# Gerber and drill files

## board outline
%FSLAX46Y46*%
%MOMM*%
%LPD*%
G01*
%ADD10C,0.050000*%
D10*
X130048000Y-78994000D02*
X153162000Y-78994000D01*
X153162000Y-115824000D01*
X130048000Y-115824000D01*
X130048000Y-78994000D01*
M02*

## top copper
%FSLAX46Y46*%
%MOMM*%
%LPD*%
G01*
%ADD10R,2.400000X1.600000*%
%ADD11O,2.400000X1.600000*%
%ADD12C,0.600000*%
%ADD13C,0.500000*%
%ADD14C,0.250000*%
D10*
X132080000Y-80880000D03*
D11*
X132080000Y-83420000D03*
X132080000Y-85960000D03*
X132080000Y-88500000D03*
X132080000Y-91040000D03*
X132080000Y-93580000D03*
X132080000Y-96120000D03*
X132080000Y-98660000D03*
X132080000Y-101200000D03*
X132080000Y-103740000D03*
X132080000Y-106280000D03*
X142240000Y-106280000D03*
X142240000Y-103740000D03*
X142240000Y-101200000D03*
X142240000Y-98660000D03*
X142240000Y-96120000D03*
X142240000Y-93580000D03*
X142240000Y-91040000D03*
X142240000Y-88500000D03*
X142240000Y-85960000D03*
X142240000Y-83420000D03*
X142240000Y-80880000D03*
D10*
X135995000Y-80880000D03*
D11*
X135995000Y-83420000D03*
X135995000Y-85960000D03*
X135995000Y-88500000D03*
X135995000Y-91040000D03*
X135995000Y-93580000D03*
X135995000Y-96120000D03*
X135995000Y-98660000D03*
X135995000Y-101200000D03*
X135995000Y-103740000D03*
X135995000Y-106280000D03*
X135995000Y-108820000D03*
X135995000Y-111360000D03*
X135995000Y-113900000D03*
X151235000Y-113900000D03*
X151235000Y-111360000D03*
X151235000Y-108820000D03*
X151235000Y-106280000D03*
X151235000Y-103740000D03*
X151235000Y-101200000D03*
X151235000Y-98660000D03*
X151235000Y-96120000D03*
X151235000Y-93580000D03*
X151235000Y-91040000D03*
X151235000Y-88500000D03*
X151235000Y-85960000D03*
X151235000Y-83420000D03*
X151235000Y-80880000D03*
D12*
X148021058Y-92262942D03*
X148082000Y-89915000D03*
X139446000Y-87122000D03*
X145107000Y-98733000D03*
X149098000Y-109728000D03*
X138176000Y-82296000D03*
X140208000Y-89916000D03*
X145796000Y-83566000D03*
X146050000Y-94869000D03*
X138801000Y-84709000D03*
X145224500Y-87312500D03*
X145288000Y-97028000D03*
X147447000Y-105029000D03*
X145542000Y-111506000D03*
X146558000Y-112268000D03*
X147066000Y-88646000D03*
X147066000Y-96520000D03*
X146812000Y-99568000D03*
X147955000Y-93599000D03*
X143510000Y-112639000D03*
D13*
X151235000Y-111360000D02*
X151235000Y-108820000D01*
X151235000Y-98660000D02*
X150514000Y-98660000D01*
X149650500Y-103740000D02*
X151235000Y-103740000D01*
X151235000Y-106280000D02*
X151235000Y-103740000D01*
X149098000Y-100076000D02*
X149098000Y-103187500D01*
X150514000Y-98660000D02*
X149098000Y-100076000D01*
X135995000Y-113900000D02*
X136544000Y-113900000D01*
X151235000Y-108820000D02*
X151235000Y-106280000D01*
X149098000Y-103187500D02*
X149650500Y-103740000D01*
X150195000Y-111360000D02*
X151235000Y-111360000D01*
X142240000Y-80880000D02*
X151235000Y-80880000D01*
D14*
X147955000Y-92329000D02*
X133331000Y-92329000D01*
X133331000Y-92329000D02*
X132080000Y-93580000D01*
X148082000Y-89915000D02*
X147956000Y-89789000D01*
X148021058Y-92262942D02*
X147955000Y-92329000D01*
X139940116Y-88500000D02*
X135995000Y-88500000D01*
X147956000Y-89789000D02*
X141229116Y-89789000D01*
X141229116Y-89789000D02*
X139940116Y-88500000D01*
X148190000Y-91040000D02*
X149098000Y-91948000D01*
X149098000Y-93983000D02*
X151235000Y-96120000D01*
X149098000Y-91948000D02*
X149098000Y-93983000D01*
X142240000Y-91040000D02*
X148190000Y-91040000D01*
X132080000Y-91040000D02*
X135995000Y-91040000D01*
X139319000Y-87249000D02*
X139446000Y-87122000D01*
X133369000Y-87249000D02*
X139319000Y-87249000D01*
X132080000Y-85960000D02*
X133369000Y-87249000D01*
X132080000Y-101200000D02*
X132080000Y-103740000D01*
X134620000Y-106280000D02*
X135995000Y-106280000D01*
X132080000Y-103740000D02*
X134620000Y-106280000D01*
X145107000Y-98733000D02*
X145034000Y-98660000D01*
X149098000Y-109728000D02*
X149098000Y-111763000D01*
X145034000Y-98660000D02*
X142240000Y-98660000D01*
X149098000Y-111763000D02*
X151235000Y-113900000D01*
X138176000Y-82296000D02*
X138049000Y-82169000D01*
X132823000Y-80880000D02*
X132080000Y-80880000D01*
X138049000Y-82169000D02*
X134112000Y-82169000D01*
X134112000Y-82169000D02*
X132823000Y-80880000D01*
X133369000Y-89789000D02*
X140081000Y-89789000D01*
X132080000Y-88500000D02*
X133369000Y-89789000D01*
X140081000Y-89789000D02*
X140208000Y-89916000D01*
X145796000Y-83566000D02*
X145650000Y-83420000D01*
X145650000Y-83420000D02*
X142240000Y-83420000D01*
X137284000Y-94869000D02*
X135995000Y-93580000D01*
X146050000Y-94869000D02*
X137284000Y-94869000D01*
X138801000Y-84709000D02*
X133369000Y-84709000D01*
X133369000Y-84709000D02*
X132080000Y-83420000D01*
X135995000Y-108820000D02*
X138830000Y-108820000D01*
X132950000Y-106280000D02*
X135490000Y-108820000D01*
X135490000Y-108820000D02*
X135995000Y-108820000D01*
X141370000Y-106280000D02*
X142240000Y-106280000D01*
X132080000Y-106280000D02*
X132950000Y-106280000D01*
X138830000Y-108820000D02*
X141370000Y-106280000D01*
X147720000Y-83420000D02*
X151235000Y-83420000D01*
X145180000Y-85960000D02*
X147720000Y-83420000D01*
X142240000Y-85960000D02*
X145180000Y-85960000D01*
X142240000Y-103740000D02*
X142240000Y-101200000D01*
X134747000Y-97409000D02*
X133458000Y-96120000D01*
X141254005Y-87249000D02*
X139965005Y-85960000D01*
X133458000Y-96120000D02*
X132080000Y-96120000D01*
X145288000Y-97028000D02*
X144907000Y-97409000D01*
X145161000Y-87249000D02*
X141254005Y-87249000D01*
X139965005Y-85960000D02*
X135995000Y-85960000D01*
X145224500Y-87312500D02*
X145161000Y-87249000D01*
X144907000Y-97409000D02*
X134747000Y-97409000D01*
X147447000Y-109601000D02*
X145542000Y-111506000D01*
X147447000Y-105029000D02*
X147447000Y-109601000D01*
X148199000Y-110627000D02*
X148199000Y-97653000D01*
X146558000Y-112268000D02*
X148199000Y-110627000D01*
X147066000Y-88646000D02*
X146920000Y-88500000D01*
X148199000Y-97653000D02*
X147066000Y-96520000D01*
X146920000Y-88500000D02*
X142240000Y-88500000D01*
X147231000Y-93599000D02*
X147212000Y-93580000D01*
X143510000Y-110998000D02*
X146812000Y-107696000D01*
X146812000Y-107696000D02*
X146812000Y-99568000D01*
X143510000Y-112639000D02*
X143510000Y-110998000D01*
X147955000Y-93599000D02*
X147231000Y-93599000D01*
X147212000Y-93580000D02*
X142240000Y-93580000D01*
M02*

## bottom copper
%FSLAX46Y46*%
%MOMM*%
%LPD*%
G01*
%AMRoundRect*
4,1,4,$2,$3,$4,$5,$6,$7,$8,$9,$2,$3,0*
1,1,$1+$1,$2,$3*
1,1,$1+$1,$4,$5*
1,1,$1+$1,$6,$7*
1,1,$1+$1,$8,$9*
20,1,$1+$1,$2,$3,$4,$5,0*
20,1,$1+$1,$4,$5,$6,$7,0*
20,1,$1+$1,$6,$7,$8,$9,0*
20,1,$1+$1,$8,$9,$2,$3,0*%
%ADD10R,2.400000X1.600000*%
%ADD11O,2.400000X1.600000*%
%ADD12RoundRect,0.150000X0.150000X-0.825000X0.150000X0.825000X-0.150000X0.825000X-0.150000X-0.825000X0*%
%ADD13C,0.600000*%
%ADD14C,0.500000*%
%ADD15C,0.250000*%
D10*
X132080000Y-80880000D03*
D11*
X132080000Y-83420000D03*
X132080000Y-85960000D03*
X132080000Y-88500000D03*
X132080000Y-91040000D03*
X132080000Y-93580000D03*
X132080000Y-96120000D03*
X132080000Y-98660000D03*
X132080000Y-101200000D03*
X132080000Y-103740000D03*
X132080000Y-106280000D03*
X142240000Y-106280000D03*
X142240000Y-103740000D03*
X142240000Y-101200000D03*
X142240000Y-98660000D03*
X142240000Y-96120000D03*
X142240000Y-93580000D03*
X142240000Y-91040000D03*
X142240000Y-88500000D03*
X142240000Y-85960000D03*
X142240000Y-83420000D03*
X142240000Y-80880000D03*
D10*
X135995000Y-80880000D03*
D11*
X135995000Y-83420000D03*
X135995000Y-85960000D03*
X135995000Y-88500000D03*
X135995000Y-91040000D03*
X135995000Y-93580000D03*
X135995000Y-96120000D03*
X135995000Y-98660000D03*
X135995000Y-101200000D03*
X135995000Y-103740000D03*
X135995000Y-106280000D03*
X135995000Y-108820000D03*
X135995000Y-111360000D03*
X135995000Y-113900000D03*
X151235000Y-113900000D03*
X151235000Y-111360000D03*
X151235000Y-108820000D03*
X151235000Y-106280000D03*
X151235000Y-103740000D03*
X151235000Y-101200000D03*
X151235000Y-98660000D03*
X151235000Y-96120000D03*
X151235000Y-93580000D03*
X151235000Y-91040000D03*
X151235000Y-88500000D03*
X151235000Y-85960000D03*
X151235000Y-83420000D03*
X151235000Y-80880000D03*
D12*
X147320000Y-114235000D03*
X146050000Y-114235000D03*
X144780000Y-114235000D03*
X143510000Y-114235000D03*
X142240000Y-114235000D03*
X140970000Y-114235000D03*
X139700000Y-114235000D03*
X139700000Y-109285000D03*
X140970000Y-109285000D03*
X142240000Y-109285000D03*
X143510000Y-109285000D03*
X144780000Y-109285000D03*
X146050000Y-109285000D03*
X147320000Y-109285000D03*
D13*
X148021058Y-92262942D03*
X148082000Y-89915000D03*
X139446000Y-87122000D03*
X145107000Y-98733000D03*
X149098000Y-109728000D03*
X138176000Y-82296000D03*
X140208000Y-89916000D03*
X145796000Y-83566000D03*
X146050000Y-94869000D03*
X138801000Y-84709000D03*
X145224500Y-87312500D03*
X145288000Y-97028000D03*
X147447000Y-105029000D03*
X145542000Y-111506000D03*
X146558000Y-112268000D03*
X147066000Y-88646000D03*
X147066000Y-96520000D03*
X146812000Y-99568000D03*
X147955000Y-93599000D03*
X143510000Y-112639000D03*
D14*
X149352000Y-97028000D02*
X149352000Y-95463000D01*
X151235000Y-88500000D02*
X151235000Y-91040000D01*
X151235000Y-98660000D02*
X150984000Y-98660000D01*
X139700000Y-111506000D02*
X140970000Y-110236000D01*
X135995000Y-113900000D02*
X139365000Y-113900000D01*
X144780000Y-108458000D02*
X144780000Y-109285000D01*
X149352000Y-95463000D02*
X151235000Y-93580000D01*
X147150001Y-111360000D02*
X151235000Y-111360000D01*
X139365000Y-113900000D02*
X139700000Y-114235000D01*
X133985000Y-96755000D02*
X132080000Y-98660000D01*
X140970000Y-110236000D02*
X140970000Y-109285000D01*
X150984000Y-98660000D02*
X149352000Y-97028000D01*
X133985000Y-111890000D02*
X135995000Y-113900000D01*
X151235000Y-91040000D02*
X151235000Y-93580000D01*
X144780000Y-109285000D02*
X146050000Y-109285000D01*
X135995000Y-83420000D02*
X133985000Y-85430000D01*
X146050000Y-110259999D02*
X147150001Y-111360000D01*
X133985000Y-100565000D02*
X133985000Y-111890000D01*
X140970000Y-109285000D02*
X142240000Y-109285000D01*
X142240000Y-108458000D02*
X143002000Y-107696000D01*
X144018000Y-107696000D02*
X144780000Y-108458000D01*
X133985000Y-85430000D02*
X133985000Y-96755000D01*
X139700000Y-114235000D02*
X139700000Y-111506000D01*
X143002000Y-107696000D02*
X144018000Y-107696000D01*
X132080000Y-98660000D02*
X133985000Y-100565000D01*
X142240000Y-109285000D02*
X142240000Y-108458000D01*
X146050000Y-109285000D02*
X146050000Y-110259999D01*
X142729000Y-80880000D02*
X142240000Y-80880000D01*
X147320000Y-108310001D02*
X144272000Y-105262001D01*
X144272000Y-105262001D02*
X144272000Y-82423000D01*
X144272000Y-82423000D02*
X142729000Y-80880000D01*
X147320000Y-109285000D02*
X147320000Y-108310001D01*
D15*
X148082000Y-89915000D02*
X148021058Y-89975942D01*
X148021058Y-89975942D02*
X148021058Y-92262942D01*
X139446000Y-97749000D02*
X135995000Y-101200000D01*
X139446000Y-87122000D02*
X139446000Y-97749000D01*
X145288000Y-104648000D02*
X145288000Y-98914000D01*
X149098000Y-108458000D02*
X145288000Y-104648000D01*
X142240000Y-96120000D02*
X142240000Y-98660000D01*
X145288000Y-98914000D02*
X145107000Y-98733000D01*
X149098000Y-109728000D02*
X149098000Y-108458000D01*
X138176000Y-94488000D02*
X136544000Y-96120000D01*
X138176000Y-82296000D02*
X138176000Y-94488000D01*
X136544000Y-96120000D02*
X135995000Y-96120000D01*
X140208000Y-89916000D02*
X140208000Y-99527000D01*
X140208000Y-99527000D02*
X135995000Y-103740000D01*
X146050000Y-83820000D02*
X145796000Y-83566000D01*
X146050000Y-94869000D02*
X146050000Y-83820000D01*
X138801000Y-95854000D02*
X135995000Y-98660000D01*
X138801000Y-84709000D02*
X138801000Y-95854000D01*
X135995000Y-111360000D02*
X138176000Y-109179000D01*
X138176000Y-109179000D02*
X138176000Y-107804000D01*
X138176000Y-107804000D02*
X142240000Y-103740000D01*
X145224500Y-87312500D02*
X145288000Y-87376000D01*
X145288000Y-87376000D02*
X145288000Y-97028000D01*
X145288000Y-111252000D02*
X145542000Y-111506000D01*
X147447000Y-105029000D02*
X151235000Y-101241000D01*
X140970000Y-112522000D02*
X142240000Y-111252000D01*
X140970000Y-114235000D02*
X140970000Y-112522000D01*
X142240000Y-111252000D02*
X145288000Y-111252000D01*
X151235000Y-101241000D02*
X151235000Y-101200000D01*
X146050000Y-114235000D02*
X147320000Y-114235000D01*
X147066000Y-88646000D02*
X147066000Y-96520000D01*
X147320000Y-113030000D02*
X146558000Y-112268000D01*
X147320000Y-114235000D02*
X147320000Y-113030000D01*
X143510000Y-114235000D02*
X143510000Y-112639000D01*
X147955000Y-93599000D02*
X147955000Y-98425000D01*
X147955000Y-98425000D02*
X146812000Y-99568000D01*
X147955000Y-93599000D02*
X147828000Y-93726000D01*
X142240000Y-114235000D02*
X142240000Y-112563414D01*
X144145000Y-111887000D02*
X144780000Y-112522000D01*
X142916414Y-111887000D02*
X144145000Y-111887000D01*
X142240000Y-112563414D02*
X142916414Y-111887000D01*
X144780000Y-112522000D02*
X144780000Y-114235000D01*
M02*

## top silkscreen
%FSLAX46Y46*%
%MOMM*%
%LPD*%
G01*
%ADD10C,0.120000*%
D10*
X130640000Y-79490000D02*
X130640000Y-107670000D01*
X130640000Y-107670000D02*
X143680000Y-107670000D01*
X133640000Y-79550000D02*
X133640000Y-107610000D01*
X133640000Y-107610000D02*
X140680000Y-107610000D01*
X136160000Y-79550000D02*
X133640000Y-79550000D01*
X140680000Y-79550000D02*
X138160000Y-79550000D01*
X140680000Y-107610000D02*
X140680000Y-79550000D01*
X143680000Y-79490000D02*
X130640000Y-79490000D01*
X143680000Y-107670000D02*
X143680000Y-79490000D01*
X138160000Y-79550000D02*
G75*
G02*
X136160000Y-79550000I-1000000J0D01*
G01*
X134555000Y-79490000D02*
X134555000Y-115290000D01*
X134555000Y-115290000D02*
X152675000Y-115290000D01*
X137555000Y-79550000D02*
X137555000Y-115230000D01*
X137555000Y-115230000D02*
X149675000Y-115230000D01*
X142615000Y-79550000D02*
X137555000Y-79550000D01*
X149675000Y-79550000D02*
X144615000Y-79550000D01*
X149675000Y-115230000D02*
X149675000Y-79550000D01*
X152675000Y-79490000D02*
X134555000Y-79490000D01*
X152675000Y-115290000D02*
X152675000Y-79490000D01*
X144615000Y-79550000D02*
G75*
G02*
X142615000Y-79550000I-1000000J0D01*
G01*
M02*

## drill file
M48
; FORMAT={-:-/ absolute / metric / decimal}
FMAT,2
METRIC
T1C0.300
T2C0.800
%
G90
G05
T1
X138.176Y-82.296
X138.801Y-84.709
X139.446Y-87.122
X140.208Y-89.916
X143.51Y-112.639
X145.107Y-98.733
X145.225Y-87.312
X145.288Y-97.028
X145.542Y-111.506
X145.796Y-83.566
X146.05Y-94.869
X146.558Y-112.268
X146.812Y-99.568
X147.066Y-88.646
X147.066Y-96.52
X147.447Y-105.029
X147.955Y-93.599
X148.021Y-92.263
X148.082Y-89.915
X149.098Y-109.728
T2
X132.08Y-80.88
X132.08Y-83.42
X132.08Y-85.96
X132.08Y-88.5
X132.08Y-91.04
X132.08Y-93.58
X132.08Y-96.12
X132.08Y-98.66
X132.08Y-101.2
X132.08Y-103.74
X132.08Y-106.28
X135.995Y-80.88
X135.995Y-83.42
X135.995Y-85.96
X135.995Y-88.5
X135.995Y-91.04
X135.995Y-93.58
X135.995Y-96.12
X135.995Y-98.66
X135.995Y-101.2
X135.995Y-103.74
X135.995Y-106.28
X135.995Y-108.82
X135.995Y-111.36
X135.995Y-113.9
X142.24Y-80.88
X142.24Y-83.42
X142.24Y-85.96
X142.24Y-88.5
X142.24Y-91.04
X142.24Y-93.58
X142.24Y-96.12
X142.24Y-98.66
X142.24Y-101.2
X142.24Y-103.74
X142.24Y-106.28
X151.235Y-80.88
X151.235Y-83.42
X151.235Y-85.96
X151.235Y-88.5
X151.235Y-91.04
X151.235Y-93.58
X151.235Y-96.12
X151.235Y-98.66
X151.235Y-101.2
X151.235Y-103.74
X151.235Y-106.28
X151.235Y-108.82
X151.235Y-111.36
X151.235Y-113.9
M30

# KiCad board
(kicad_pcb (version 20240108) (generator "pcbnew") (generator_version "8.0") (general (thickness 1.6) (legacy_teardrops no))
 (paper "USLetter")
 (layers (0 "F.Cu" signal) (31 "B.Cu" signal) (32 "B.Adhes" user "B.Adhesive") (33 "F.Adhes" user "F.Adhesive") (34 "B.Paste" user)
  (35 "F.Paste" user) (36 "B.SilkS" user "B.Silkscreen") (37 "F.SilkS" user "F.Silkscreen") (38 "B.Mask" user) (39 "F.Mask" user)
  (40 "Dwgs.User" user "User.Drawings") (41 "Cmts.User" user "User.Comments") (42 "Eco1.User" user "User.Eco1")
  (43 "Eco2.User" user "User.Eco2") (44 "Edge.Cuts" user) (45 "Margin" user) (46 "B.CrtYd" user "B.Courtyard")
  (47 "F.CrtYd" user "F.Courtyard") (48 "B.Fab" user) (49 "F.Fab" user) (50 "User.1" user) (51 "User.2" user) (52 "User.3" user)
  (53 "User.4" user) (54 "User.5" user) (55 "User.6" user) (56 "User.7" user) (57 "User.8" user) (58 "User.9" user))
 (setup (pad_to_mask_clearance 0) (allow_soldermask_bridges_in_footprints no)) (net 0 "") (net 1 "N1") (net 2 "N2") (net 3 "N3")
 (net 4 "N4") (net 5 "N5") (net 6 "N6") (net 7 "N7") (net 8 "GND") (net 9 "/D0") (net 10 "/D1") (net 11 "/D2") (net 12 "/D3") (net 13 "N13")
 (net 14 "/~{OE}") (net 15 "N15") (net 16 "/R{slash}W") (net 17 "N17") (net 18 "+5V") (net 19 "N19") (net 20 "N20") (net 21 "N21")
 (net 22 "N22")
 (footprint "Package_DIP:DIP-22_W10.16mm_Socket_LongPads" (layer "F.Cu") (at 132.08 80.88)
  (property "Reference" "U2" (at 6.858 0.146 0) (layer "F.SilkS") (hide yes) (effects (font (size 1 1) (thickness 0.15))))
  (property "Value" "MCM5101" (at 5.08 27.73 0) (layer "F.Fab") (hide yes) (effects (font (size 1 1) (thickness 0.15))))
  (fp_line (start -1.44 -1.39) (end -1.44 26.79) (stroke (width 0.12) (type solid)) (layer "F.SilkS"))
  (fp_line (start -1.44 26.79) (end 11.6 26.79) (stroke (width 0.12) (type solid)) (layer "F.SilkS"))
  (fp_line (start 1.56 -1.33) (end 1.56 26.73) (stroke (width 0.12) (type solid)) (layer "F.SilkS"))
  (fp_line (start 1.56 26.73) (end 8.6 26.73) (stroke (width 0.12) (type solid)) (layer "F.SilkS"))
  (fp_line (start 4.08 -1.33) (end 1.56 -1.33) (stroke (width 0.12) (type solid)) (layer "F.SilkS"))
  (fp_line (start 8.6 -1.33) (end 6.08 -1.33) (stroke (width 0.12) (type solid)) (layer "F.SilkS"))
  (fp_line (start 8.6 26.73) (end 8.6 -1.33) (stroke (width 0.12) (type solid)) (layer "F.SilkS"))
  (fp_line (start 11.6 -1.39) (end -1.44 -1.39) (stroke (width 0.12) (type solid)) (layer "F.SilkS"))
  (fp_line (start 11.6 26.79) (end 11.6 -1.39) (stroke (width 0.12) (type solid)) (layer "F.SilkS"))
  (fp_arc (start 6.08 -1.33) (mid 5.08 -0.33) (end 4.08 -1.33) (stroke (width 0.12) (type solid)) (layer "F.SilkS"))
  (pad "1" thru_hole rect (at 0 0) (size 2.4 1.6) (drill 0.8) (layers "*.Cu" "*.Mask") (remove_unused_layers no) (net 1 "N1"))
  (pad "2" thru_hole oval (at 0 2.54) (size 2.4 1.6) (drill 0.8) (layers "*.Cu" "*.Mask") (remove_unused_layers no) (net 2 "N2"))
  (pad "3" thru_hole oval (at 0 5.08) (size 2.4 1.6) (drill 0.8) (layers "*.Cu" "*.Mask") (remove_unused_layers no) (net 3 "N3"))
  (pad "4" thru_hole oval (at 0 7.62) (size 2.4 1.6) (drill 0.8) (layers "*.Cu" "*.Mask") (remove_unused_layers no) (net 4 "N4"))
  (pad "5" thru_hole oval (at 0 10.16) (size 2.4 1.6) (drill 0.8) (layers "*.Cu" "*.Mask") (remove_unused_layers no) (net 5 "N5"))
  (pad "6" thru_hole oval (at 0 12.7) (size 2.4 1.6) (drill 0.8) (layers "*.Cu" "*.Mask") (remove_unused_layers no) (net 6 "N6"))
  (pad "7" thru_hole oval (at 0 15.24) (size 2.4 1.6) (drill 0.8) (layers "*.Cu" "*.Mask") (remove_unused_layers no) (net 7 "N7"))
  (pad "8" thru_hole oval (at 0 17.78) (size 2.4 1.6) (drill 0.8) (layers "*.Cu" "*.Mask") (remove_unused_layers no) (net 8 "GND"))
  (pad "9" thru_hole oval (at 0 20.32) (size 2.4 1.6) (drill 0.8) (layers "*.Cu" "*.Mask") (remove_unused_layers no) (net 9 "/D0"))
  (pad "10" thru_hole oval (at 0 22.86) (size 2.4 1.6) (drill 0.8) (layers "*.Cu" "*.Mask") (remove_unused_layers no) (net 9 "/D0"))
  (pad "11" thru_hole oval (at 0 25.4) (size 2.4 1.6) (drill 0.8) (layers "*.Cu" "*.Mask") (remove_unused_layers no) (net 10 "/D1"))
  (pad "12" thru_hole oval (at 10.16 25.4) (size 2.4 1.6) (drill 0.8) (layers "*.Cu" "*.Mask") (remove_unused_layers no) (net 10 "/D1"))
  (pad "13" thru_hole oval (at 10.16 22.86) (size 2.4 1.6) (drill 0.8) (layers "*.Cu" "*.Mask") (remove_unused_layers no) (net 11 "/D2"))
  (pad "14" thru_hole oval (at 10.16 20.32) (size 2.4 1.6) (drill 0.8) (layers "*.Cu" "*.Mask") (remove_unused_layers no) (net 11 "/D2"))
  (pad "15" thru_hole oval (at 10.16 17.78) (size 2.4 1.6) (drill 0.8) (layers "*.Cu" "*.Mask") (remove_unused_layers no) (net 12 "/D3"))
  (pad "16" thru_hole oval (at 10.16 15.24) (size 2.4 1.6) (drill 0.8) (layers "*.Cu" "*.Mask") (remove_unused_layers no) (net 12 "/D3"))
  (pad "17" thru_hole oval (at 10.16 12.7) (size 2.4 1.6) (drill 0.8) (layers "*.Cu" "*.Mask") (remove_unused_layers no) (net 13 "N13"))
  (pad "18" thru_hole oval (at 10.16 10.16) (size 2.4 1.6) (drill 0.8) (layers "*.Cu" "*.Mask") (remove_unused_layers no) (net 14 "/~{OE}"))
  (pad "19" thru_hole oval (at 10.16 7.62) (size 2.4 1.6) (drill 0.8) (layers "*.Cu" "*.Mask") (remove_unused_layers no) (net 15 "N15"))
  (pad "20" thru_hole oval (at 10.16 5.08) (size 2.4 1.6) (drill 0.8) (layers "*.Cu" "*.Mask") (remove_unused_layers no)
   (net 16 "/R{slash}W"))
  (pad "21" thru_hole oval (at 10.16 2.54) (size 2.4 1.6) (drill 0.8) (layers "*.Cu" "*.Mask") (remove_unused_layers no) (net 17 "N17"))
  (pad "22" thru_hole oval (at 10.16 0) (size 2.4 1.6) (drill 0.8) (layers "*.Cu" "*.Mask") (remove_unused_layers no) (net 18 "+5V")))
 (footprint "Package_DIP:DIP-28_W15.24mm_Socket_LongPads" (layer "F.Cu") (at 135.995 80.88)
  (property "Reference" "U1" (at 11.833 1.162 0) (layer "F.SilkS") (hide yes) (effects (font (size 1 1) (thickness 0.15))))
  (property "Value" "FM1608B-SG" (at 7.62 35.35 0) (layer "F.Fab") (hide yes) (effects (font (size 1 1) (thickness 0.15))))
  (fp_line (start -1.44 -1.39) (end -1.44 34.41) (stroke (width 0.12) (type solid)) (layer "F.SilkS"))
  (fp_line (start -1.44 34.41) (end 16.68 34.41) (stroke (width 0.12) (type solid)) (layer "F.SilkS"))
  (fp_line (start 1.56 -1.33) (end 1.56 34.35) (stroke (width 0.12) (type solid)) (layer "F.SilkS"))
  (fp_line (start 1.56 34.35) (end 13.68 34.35) (stroke (width 0.12) (type solid)) (layer "F.SilkS"))
  (fp_line (start 6.62 -1.33) (end 1.56 -1.33) (stroke (width 0.12) (type solid)) (layer "F.SilkS"))
  (fp_line (start 13.68 -1.33) (end 8.62 -1.33) (stroke (width 0.12) (type solid)) (layer "F.SilkS"))
  (fp_line (start 13.68 34.35) (end 13.68 -1.33) (stroke (width 0.12) (type solid)) (layer "F.SilkS"))
  (fp_line (start 16.68 -1.39) (end -1.44 -1.39) (stroke (width 0.12) (type solid)) (layer "F.SilkS"))
  (fp_line (start 16.68 34.41) (end 16.68 -1.39) (stroke (width 0.12) (type solid)) (layer "F.SilkS"))
  (fp_arc (start 8.62 -1.33) (mid 7.62 -0.33) (end 6.62 -1.33) (stroke (width 0.12) (type solid)) (layer "F.SilkS"))
  (pad "1" thru_hole rect (at 0 0) (size 2.4 1.6) (drill 0.8) (layers "*.Cu" "*.Mask") (remove_unused_layers no))
  (pad "2" thru_hole oval (at 0 2.54) (size 2.4 1.6) (drill 0.8) (layers "*.Cu" "*.Mask") (remove_unused_layers no) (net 8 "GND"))
  (pad "3" thru_hole oval (at 0 5.08) (size 2.4 1.6) (drill 0.8) (layers "*.Cu" "*.Mask") (remove_unused_layers no) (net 7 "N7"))
  (pad "4" thru_hole oval (at 0 7.62) (size 2.4 1.6) (drill 0.8) (layers "*.Cu" "*.Mask") (remove_unused_layers no) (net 6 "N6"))
  (pad "5" thru_hole oval (at 0 10.16) (size 2.4 1.6) (drill 0.8) (layers "*.Cu" "*.Mask") (remove_unused_layers no) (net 5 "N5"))
  (pad "6" thru_hole oval (at 0 12.7) (size 2.4 1.6) (drill 0.8) (layers "*.Cu" "*.Mask") (remove_unused_layers no) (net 17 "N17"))
  (pad "7" thru_hole oval (at 0 15.24) (size 2.4 1.6) (drill 0.8) (layers "*.Cu" "*.Mask") (remove_unused_layers no) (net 1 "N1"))
  (pad "8" thru_hole oval (at 0 17.78) (size 2.4 1.6) (drill 0.8) (layers "*.Cu" "*.Mask") (remove_unused_layers no) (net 2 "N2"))
  (pad "9" thru_hole oval (at 0 20.32) (size 2.4 1.6) (drill 0.8) (layers "*.Cu" "*.Mask") (remove_unused_layers no) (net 3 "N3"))
  (pad "10" thru_hole oval (at 0 22.86) (size 2.4 1.6) (drill 0.8) (layers "*.Cu" "*.Mask") (remove_unused_layers no) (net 4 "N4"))
  (pad "11" thru_hole oval (at 0 25.4) (size 2.4 1.6) (drill 0.8) (layers "*.Cu" "*.Mask") (remove_unused_layers no) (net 9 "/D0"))
  (pad "12" thru_hole oval (at 0 27.94) (size 2.4 1.6) (drill 0.8) (layers "*.Cu" "*.Mask") (remove_unused_layers no) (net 10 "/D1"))
  (pad "13" thru_hole oval (at 0 30.48) (size 2.4 1.6) (drill 0.8) (layers "*.Cu" "*.Mask") (remove_unused_layers no) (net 11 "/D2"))
  (pad "14" thru_hole oval (at 0 33.02) (size 2.4 1.6) (drill 0.8) (layers "*.Cu" "*.Mask") (remove_unused_layers no) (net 8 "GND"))
  (pad "15" thru_hole oval (at 15.24 33.02) (size 2.4 1.6) (drill 0.8) (layers "*.Cu" "*.Mask") (remove_unused_layers no) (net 12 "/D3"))
  (pad "16" thru_hole oval (at 15.24 30.48) (size 2.4 1.6) (drill 0.8) (layers "*.Cu" "*.Mask") (remove_unused_layers no) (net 8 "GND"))
  (pad "17" thru_hole oval (at 15.24 27.94) (size 2.4 1.6) (drill 0.8) (layers "*.Cu" "*.Mask") (remove_unused_layers no) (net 8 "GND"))
  (pad "18" thru_hole oval (at 15.24 25.4) (size 2.4 1.6) (drill 0.8) (layers "*.Cu" "*.Mask") (remove_unused_layers no) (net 8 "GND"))
  (pad "19" thru_hole oval (at 15.24 22.86) (size 2.4 1.6) (drill 0.8) (layers "*.Cu" "*.Mask") (remove_unused_layers no) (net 8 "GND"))
  (pad "20" thru_hole oval (at 15.24 20.32) (size 2.4 1.6) (drill 0.8) (layers "*.Cu" "*.Mask") (remove_unused_layers no) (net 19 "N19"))
  (pad "21" thru_hole oval (at 15.24 17.78) (size 2.4 1.6) (drill 0.8) (layers "*.Cu" "*.Mask") (remove_unused_layers no) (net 8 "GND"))
  (pad "22" thru_hole oval (at 15.24 15.24) (size 2.4 1.6) (drill 0.8) (layers "*.Cu" "*.Mask") (remove_unused_layers no) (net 14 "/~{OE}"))
  (pad "23" thru_hole oval (at 15.24 12.7) (size 2.4 1.6) (drill 0.8) (layers "*.Cu" "*.Mask") (remove_unused_layers no) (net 8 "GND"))
  (pad "24" thru_hole oval (at 15.24 10.16) (size 2.4 1.6) (drill 0.8) (layers "*.Cu" "*.Mask") (remove_unused_layers no) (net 8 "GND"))
  (pad "25" thru_hole oval (at 15.24 7.62) (size 2.4 1.6) (drill 0.8) (layers "*.Cu" "*.Mask") (remove_unused_layers no) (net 8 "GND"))
  (pad "26" thru_hole oval (at 15.24 5.08) (size 2.4 1.6) (drill 0.8) (layers "*.Cu" "*.Mask") (remove_unused_layers no))
  (pad "27" thru_hole oval (at 15.24 2.54) (size 2.4 1.6) (drill 0.8) (layers "*.Cu" "*.Mask") (remove_unused_layers no)
   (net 16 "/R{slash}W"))
  (pad "28" thru_hole oval (at 15.24 0) (size 2.4 1.6) (drill 0.8) (layers "*.Cu" "*.Mask") (remove_unused_layers no) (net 18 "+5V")))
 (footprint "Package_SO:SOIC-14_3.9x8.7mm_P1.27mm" (layer "B.Cu") (at 143.51 111.76 90)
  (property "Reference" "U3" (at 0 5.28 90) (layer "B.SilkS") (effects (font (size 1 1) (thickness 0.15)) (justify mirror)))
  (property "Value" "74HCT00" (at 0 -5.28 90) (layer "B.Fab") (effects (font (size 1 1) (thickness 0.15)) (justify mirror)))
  (pad "1" smd roundrect (at -2.475 3.81 90) (size 1.95 0.6) (layers "B.Cu" "B.Paste" "B.Mask") (roundrect_rratio 0.25) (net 15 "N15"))
  (pad "2" smd roundrect (at -2.475 2.54 90) (size 1.95 0.6) (layers "B.Cu" "B.Paste" "B.Mask") (roundrect_rratio 0.25) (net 15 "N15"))
  (pad "3" smd roundrect (at -2.475 1.27 90) (size 1.95 0.6) (layers "B.Cu" "B.Paste" "B.Mask") (roundrect_rratio 0.25) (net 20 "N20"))
  (pad "4" smd roundrect (at -2.475 0 90) (size 1.95 0.6) (layers "B.Cu" "B.Paste" "B.Mask") (roundrect_rratio 0.25) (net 13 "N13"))
  (pad "5" smd roundrect (at -2.475 -1.27 90) (size 1.95 0.6) (layers "B.Cu" "B.Paste" "B.Mask") (roundrect_rratio 0.25) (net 20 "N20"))
  (pad "6" smd roundrect (at -2.475 -2.54 90) (size 1.95 0.6) (layers "B.Cu" "B.Paste" "B.Mask") (roundrect_rratio 0.25) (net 19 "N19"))
  (pad "7" smd roundrect (at -2.475 -3.81 90) (size 1.95 0.6) (layers "B.Cu" "B.Paste" "B.Mask") (roundrect_rratio 0.25) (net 8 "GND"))
  (pad "8" smd roundrect (at 2.475 -3.81 90) (size 1.95 0.6) (layers "B.Cu" "B.Paste" "B.Mask") (roundrect_rratio 0.25) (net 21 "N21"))
  (pad "9" smd roundrect (at 2.475 -2.54 90) (size 1.95 0.6) (layers "B.Cu" "B.Paste" "B.Mask") (roundrect_rratio 0.25) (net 8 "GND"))
  (pad "10" smd roundrect (at 2.475 -1.27 90) (size 1.95 0.6) (layers "B.Cu" "B.Paste" "B.Mask") (roundrect_rratio 0.25) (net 8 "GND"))
  (pad "11" smd roundrect (at 2.475 0 90) (size 1.95 0.6) (layers "B.Cu" "B.Paste" "B.Mask") (roundrect_rratio 0.25) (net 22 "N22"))
  (pad "12" smd roundrect (at 2.475 1.27 90) (size 1.95 0.6) (layers "B.Cu" "B.Paste" "B.Mask") (roundrect_rratio 0.25) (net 8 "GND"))
  (pad "13" smd roundrect (at 2.475 2.54 90) (size 1.95 0.6) (layers "B.Cu" "B.Paste" "B.Mask") (roundrect_rratio 0.25) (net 8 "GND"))
  (pad "14" smd roundrect (at 2.475 3.81 90) (size 1.95 0.6) (layers "B.Cu" "B.Paste" "B.Mask") (roundrect_rratio 0.25) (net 18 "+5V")))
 (gr_rect (start 130.048 78.994) (end 153.162 115.824) (stroke (width 0.05) (type default)) (fill none) (layer "Edge.Cuts"))
 (segment (start 151.235 111.36) (end 151.235 108.82) (width 0.5) (layer "F.Cu") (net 8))
 (segment (start 151.235 98.66) (end 150.514 98.66) (width 0.5) (layer "F.Cu") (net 8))
 (segment (start 149.6505 103.74) (end 151.235 103.74) (width 0.5) (layer "F.Cu") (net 8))
 (segment (start 151.235 106.28) (end 151.235 103.74) (width 0.5) (layer "F.Cu") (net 8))
 (segment (start 149.098 100.076) (end 149.098 103.1875) (width 0.5) (layer "F.Cu") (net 8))
 (segment (start 150.514 98.66) (end 149.098 100.076) (width 0.5) (layer "F.Cu") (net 8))
 (segment (start 135.995 113.9) (end 136.544 113.9) (width 0.5) (layer "F.Cu") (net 8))
 (segment (start 151.235 108.82) (end 151.235 106.28) (width 0.5) (layer "F.Cu") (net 8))
 (segment (start 149.098 103.1875) (end 149.6505 103.74) (width 0.5) (layer "F.Cu") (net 8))
 (segment (start 150.195 111.36) (end 151.235 111.36) (width 0.5) (layer "F.Cu") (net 8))
 (segment (start 149.352 97.028) (end 149.352 95.463) (width 0.5) (layer "B.Cu") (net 8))
 (segment (start 151.235 88.5) (end 151.235 91.04) (width 0.5) (layer "B.Cu") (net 8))
 (segment (start 151.235 98.66) (end 150.984 98.66) (width 0.5) (layer "B.Cu") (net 8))
 (segment (start 139.7 111.506) (end 140.97 110.236) (width 0.5) (layer "B.Cu") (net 8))
 (segment (start 135.995 113.9) (end 139.365 113.9) (width 0.5) (layer "B.Cu") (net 8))
 (segment (start 144.78 108.458) (end 144.78 109.285) (width 0.5) (layer "B.Cu") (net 8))
 (segment (start 149.352 95.463) (end 151.235 93.58) (width 0.5) (layer "B.Cu") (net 8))
 (segment (start 147.150001 111.36) (end 151.235 111.36) (width 0.5) (layer "B.Cu") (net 8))
 (segment (start 139.365 113.9) (end 139.7 114.235) (width 0.5) (layer "B.Cu") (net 8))
 (segment (start 133.985 96.755) (end 132.08 98.66) (width 0.5) (layer "B.Cu") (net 8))
 (segment (start 140.97 110.236) (end 140.97 109.285) (width 0.5) (layer "B.Cu") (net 8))
 (segment (start 150.984 98.66) (end 149.352 97.028) (width 0.5) (layer "B.Cu") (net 8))
 (segment (start 133.985 111.89) (end 135.995 113.9) (width 0.5) (layer "B.Cu") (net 8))
 (segment (start 151.235 91.04) (end 151.235 93.58) (width 0.5) (layer "B.Cu") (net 8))
 (segment (start 144.78 109.285) (end 146.05 109.285) (width 0.5) (layer "B.Cu") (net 8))
 (segment (start 135.995 83.42) (end 133.985 85.43) (width 0.5) (layer "B.Cu") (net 8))
 (segment (start 146.05 110.259999) (end 147.150001 111.36) (width 0.5) (layer "B.Cu") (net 8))
 (segment (start 133.985 100.565) (end 133.985 111.89) (width 0.5) (layer "B.Cu") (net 8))
 (segment (start 140.97 109.285) (end 142.24 109.285) (width 0.5) (layer "B.Cu") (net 8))
 (segment (start 142.24 108.458) (end 143.002 107.696) (width 0.5) (layer "B.Cu") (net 8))
 (segment (start 144.018 107.696) (end 144.78 108.458) (width 0.5) (layer "B.Cu") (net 8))
 (segment (start 133.985 85.43) (end 133.985 96.755) (width 0.5) (layer "B.Cu") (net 8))
 (segment (start 139.7 114.235) (end 139.7 111.506) (width 0.5) (layer "B.Cu") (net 8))
 (segment (start 143.002 107.696) (end 144.018 107.696) (width 0.5) (layer "B.Cu") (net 8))
 (segment (start 132.08 98.66) (end 133.985 100.565) (width 0.5) (layer "B.Cu") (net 8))
 (segment (start 142.24 109.285) (end 142.24 108.458) (width 0.5) (layer "B.Cu") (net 8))
 (segment (start 146.05 109.285) (end 146.05 110.259999) (width 0.5) (layer "B.Cu") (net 8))
 (segment (start 142.24 80.88) (end 151.235 80.88) (width 0.5) (layer "F.Cu") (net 18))
 (segment (start 142.729 80.88) (end 142.24 80.88) (width 0.5) (layer "B.Cu") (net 18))
 (segment (start 147.32 108.310001) (end 144.272 105.262001) (width 0.5) (layer "B.Cu") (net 18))
 (segment (start 144.272 105.262001) (end 144.272 82.423) (width 0.5) (layer "B.Cu") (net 18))
 (segment (start 144.272 82.423) (end 142.729 80.88) (width 0.5) (layer "B.Cu") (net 18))
 (segment (start 147.32 109.285) (end 147.32 108.310001) (width 0.5) (layer "B.Cu") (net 18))
 (segment (start 147.955 92.329) (end 133.331 92.329) (width 0.25) (layer "F.Cu") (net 6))
 (segment (start 133.331 92.329) (end 132.08 93.58) (width 0.25) (layer "F.Cu") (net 6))
 (segment (start 148.082 89.915) (end 147.956 89.789) (width 0.25) (layer "F.Cu") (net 6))
 (segment (start 148.021058 92.262942) (end 147.955 92.329) (width 0.25) (layer "F.Cu") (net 6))
 (segment (start 139.940116 88.5) (end 135.995 88.5) (width 0.25) (layer "F.Cu") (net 6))
 (segment (start 147.956 89.789) (end 141.229116 89.789) (width 0.25) (layer "F.Cu") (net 6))
 (segment (start 141.229116 89.789) (end 139.940116 88.5) (width 0.25) (layer "F.Cu") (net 6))
 (via (at 148.021058 92.262942) (size 0.6) (drill 0.3) (layers "F.Cu" "B.Cu") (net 6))
 (via (at 148.082 89.915) (size 0.6) (drill 0.3) (layers "F.Cu" "B.Cu") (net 6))
 (segment (start 148.082 89.915) (end 148.021058 89.975942) (width 0.25) (layer "B.Cu") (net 6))
 (segment (start 148.021058 89.975942) (end 148.021058 92.262942) (width 0.25) (layer "B.Cu") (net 6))
 (segment (start 148.19 91.04) (end 149.098 91.948) (width 0.25) (layer "F.Cu") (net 14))
 (segment (start 149.098 93.983) (end 151.235 96.12) (width 0.25) (layer "F.Cu") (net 14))
 (segment (start 149.098 91.948) (end 149.098 93.983) (width 0.25) (layer "F.Cu") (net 14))
 (segment (start 142.24 91.04) (end 148.19 91.04) (width 0.25) (layer "F.Cu") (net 14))
 (segment (start 132.08 91.04) (end 135.995 91.04) (width 0.25) (layer "F.Cu") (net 5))
 (segment (start 139.319 87.249) (end 139.446 87.122) (width 0.25) (layer "F.Cu") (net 3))
 (segment (start 133.369 87.249) (end 139.319 87.249) (width 0.25) (layer "F.Cu") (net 3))
 (segment (start 132.08 85.96) (end 133.369 87.249) (width 0.25) (layer "F.Cu") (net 3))
 (via (at 139.446 87.122) (size 0.6) (drill 0.3) (layers "F.Cu" "B.Cu") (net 3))
 (segment (start 139.446 97.749) (end 135.995 101.2) (width 0.25) (layer "B.Cu") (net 3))
 (segment (start 139.446 87.122) (end 139.446 97.749) (width 0.25) (layer "B.Cu") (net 3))
 (segment (start 132.08 101.2) (end 132.08 103.74) (width 0.25) (layer "F.Cu") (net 9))
 (segment (start 134.62 106.28) (end 135.995 106.28) (width 0.25) (layer "F.Cu") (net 9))
 (segment (start 132.08 103.74) (end 134.62 106.28) (width 0.25) (layer "F.Cu") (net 9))
 (segment (start 145.107 98.733) (end 145.034 98.66) (width 0.25) (layer "F.Cu") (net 12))
 (segment (start 149.098 109.728) (end 149.098 111.763) (width 0.25) (layer "F.Cu") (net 12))
 (segment (start 145.034 98.66) (end 142.24 98.66) (width 0.25) (layer "F.Cu") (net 12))
 (segment (start 149.098 111.763) (end 151.235 113.9) (width 0.25) (layer "F.Cu") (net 12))
 (via (at 145.107 98.733) (size 0.6) (drill 0.3) (layers "F.Cu" "B.Cu") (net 12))
 (via (at 149.098 109.728) (size 0.6) (drill 0.3) (layers "F.Cu" "B.Cu") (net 12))
 (segment (start 145.288 104.648) (end 145.288 98.914) (width 0.25) (layer "B.Cu") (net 12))
 (segment (start 149.098 108.458) (end 145.288 104.648) (width 0.25) (layer "B.Cu") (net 12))
 (segment (start 142.24 96.12) (end 142.24 98.66) (width 0.25) (layer "B.Cu") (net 12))
 (segment (start 145.288 98.914) (end 145.107 98.733) (width 0.25) (layer "B.Cu") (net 12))
 (segment (start 149.098 109.728) (end 149.098 108.458) (width 0.25) (layer "B.Cu") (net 12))
 (segment (start 138.176 82.296) (end 138.049 82.169) (width 0.25) (layer "F.Cu") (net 1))
 (segment (start 132.823 80.88) (end 132.08 80.88) (width 0.25) (layer "F.Cu") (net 1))
 (segment (start 138.049 82.169) (end 134.112 82.169) (width 0.25) (layer "F.Cu") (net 1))
 (segment (start 134.112 82.169) (end 132.823 80.88) (width 0.25) (layer "F.Cu") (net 1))
 (via (at 138.176 82.296) (size 0.6) (drill 0.3) (layers "F.Cu" "B.Cu") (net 1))
 (segment (start 138.176 94.488) (end 136.544 96.12) (width 0.25) (layer "B.Cu") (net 1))
 (segment (start 138.176 82.296) (end 138.176 94.488) (width 0.25) (layer "B.Cu") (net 1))
 (segment (start 136.544 96.12) (end 135.995 96.12) (width 0.25) (layer "B.Cu") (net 1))
 (segment (start 133.369 89.789) (end 140.081 89.789) (width 0.25) (layer "F.Cu") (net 4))
 (segment (start 132.08 88.5) (end 133.369 89.789) (width 0.25) (layer "F.Cu") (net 4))
 (segment (start 140.081 89.789) (end 140.208 89.916) (width 0.25) (layer "F.Cu") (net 4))
 (via (at 140.208 89.916) (size 0.6) (drill 0.3) (layers "F.Cu" "B.Cu") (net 4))
 (segment (start 140.208 89.916) (end 140.208 99.527) (width 0.25) (layer "B.Cu") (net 4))
 (segment (start 140.208 99.527) (end 135.995 103.74) (width 0.25) (layer "B.Cu") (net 4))
 (segment (start 145.796 83.566) (end 145.65 83.42) (width 0.25) (layer "F.Cu") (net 17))
 (segment (start 145.65 83.42) (end 142.24 83.42) (width 0.25) (layer "F.Cu") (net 17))
 (segment (start 137.284 94.869) (end 135.995 93.58) (width 0.25) (layer "F.Cu") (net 17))
 (segment (start 146.05 94.869) (end 137.284 94.869) (width 0.25) (layer "F.Cu") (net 17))
 (via (at 145.796 83.566) (size 0.6) (drill 0.3) (layers "F.Cu" "B.Cu") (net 17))
 (via (at 146.05 94.869) (size 0.6) (drill 0.3) (layers "F.Cu" "B.Cu") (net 17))
 (segment (start 146.05 83.82) (end 145.796 83.566) (width 0.25) (layer "B.Cu") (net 17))
 (segment (start 146.05 94.869) (end 146.05 83.82) (width 0.25) (layer "B.Cu") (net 17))
 (segment (start 138.801 84.709) (end 133.369 84.709) (width 0.25) (layer "F.Cu") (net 2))
 (segment (start 133.369 84.709) (end 132.08 83.42) (width 0.25) (layer "F.Cu") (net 2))
 (via (at 138.801 84.709) (size 0.6) (drill 0.3) (layers "F.Cu" "B.Cu") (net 2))
 (segment (start 138.801 95.854) (end 135.995 98.66) (width 0.25) (layer "B.Cu") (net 2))
 (segment (start 138.801 84.709) (end 138.801 95.854) (width 0.25) (layer "B.Cu") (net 2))
 (segment (start 135.995 108.82) (end 138.83 108.82) (width 0.25) (layer "F.Cu") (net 10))
 (segment (start 132.95 106.28) (end 135.49 108.82) (width 0.25) (layer "F.Cu") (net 10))
 (segment (start 135.49 108.82) (end 135.995 108.82) (width 0.25) (layer "F.Cu") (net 10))
 (segment (start 141.37 106.28) (end 142.24 106.28) (width 0.25) (layer "F.Cu") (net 10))
 (segment (start 132.08 106.28) (end 132.95 106.28) (width 0.25) (layer "F.Cu") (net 10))
 (segment (start 138.83 108.82) (end 141.37 106.28) (width 0.25) (layer "F.Cu") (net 10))
 (segment (start 147.72 83.42) (end 151.235 83.42) (width 0.25) (layer "F.Cu") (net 16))
 (segment (start 145.18 85.96) (end 147.72 83.42) (width 0.25) (layer "F.Cu") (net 16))
 (segment (start 142.24 85.96) (end 145.18 85.96) (width 0.25) (layer "F.Cu") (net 16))
 (segment (start 142.24 103.74) (end 142.24 101.2) (width 0.25) (layer "F.Cu") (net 11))
 (segment (start 135.995 111.36) (end 138.176 109.179) (width 0.25) (layer "B.Cu") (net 11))
 (segment (start 138.176 109.179) (end 138.176 107.804) (width 0.25) (layer "B.Cu") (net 11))
 (segment (start 138.176 107.804) (end 142.24 103.74) (width 0.25) (layer "B.Cu") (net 11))
 (segment (start 134.747 97.409) (end 133.458 96.12) (width 0.25) (layer "F.Cu") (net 7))
 (segment (start 141.254005 87.249) (end 139.965005 85.96) (width 0.25) (layer "F.Cu") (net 7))
 (segment (start 133.458 96.12) (end 132.08 96.12) (width 0.25) (layer "F.Cu") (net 7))
 (segment (start 145.288 97.028) (end 144.907 97.409) (width 0.25) (layer "F.Cu") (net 7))
 (segment (start 145.161 87.249) (end 141.254005 87.249) (width 0.25) (layer "F.Cu") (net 7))
 (segment (start 139.965005 85.96) (end 135.995 85.96) (width 0.25) (layer "F.Cu") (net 7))
 (segment (start 145.2245 87.3125) (end 145.161 87.249) (width 0.25) (layer "F.Cu") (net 7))
 (segment (start 144.907 97.409) (end 134.747 97.409) (width 0.25) (layer "F.Cu") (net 7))
 (via (at 145.2245 87.3125) (size 0.6) (drill 0.3) (layers "F.Cu" "B.Cu") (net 7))
 (via (at 145.288 97.028) (size 0.6) (drill 0.3) (layers "F.Cu" "B.Cu") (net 7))
 (segment (start 145.2245 87.3125) (end 145.288 87.376) (width 0.25) (layer "B.Cu") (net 7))
 (segment (start 145.288 87.376) (end 145.288 97.028) (width 0.25) (layer "B.Cu") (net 7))
 (segment (start 147.447 109.601) (end 145.542 111.506) (width 0.25) (layer "F.Cu") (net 19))
 (segment (start 147.447 105.029) (end 147.447 109.601) (width 0.25) (layer "F.Cu") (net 19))
 (via (at 147.447 105.029) (size 0.6) (drill 0.3) (layers "F.Cu" "B.Cu") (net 19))
 (via (at 145.542 111.506) (size 0.6) (drill 0.3) (layers "F.Cu" "B.Cu") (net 19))
 (segment (start 145.288 111.252) (end 145.542 111.506) (width 0.25) (layer "B.Cu") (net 19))
 (segment (start 147.447 105.029) (end 151.235 101.241) (width 0.25) (layer "B.Cu") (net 19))
 (segment (start 140.97 112.522) (end 142.24 111.252) (width 0.25) (layer "B.Cu") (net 19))
 (segment (start 140.97 114.235) (end 140.97 112.522) (width 0.25) (layer "B.Cu") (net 19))
 (segment (start 142.24 111.252) (end 145.288 111.252) (width 0.25) (layer "B.Cu") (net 19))
 (segment (start 151.235 101.241) (end 151.235 101.2) (width 0.25) (layer "B.Cu") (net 19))
 (segment (start 148.199 110.627) (end 148.199 97.653) (width 0.25) (layer "F.Cu") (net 15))
 (segment (start 146.558 112.268) (end 148.199 110.627) (width 0.25) (layer "F.Cu") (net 15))
 (segment (start 147.066 88.646) (end 146.92 88.5) (width 0.25) (layer "F.Cu") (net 15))
 (segment (start 148.199 97.653) (end 147.066 96.52) (width 0.25) (layer "F.Cu") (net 15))
 (segment (start 146.92 88.5) (end 142.24 88.5) (width 0.25) (layer "F.Cu") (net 15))
 (via (at 146.558 112.268) (size 0.6) (drill 0.3) (layers "F.Cu" "B.Cu") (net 15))
 (via (at 147.066 88.646) (size 0.6) (drill 0.3) (layers "F.Cu" "B.Cu") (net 15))
 (via (at 147.066 96.52) (size 0.6) (drill 0.3) (layers "F.Cu" "B.Cu") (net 15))
 (segment (start 146.05 114.235) (end 147.32 114.235) (width 0.25) (layer "B.Cu") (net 15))
 (segment (start 147.066 88.646) (end 147.066 96.52) (width 0.25) (layer "B.Cu") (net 15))
 (segment (start 147.32 113.03) (end 146.558 112.268) (width 0.25) (layer "B.Cu") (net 15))
 (segment (start 147.32 114.235) (end 147.32 113.03) (width 0.25) (layer "B.Cu") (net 15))
 (segment (start 147.231 93.599) (end 147.212 93.58) (width 0.25) (layer "F.Cu") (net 13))
 (segment (start 143.51 110.998) (end 146.812 107.696) (width 0.25) (layer "F.Cu") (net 13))
 (segment (start 146.812 107.696) (end 146.812 99.568) (width 0.25) (layer "F.Cu") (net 13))
 (segment (start 143.51 112.639) (end 143.51 110.998) (width 0.25) (layer "F.Cu") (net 13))
 (segment (start 147.955 93.599) (end 147.231 93.599) (width 0.25) (layer "F.Cu") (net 13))
 (segment (start 147.212 93.58) (end 142.24 93.58) (width 0.25) (layer "F.Cu") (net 13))
 (via (at 146.812 99.568) (size 0.6) (drill 0.3) (layers "F.Cu" "B.Cu") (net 13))
 (via (at 147.955 93.599) (size 0.6) (drill 0.3) (layers "F.Cu" "B.Cu") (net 13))
 (via (at 143.51 112.639) (size 0.6) (drill 0.3) (layers "F.Cu" "B.Cu") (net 13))
 (segment (start 143.51 114.235) (end 143.51 112.639) (width 0.25) (layer "B.Cu") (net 13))
 (segment (start 147.955 93.599) (end 147.955 98.425) (width 0.25) (layer "B.Cu") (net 13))
 (segment (start 147.955 98.425) (end 146.812 99.568) (width 0.25) (layer "B.Cu") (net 13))
 (segment (start 147.955 93.599) (end 147.828 93.726) (width 0.25) (layer "B.Cu") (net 13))
 (segment (start 142.24 114.235) (end 142.24 112.563414) (width 0.25) (layer "B.Cu") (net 20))
 (segment (start 144.145 111.887) (end 144.78 112.522) (width 0.25) (layer "B.Cu") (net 20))
 (segment (start 142.916414 111.887) (end 144.145 111.887) (width 0.25) (layer "B.Cu") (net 20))
 (segment (start 142.24 112.563414) (end 142.916414 111.887) (width 0.25) (layer "B.Cu") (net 20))
 (segment (start 144.78 112.522) (end 144.78 114.235) (width 0.25) (layer "B.Cu") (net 20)))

